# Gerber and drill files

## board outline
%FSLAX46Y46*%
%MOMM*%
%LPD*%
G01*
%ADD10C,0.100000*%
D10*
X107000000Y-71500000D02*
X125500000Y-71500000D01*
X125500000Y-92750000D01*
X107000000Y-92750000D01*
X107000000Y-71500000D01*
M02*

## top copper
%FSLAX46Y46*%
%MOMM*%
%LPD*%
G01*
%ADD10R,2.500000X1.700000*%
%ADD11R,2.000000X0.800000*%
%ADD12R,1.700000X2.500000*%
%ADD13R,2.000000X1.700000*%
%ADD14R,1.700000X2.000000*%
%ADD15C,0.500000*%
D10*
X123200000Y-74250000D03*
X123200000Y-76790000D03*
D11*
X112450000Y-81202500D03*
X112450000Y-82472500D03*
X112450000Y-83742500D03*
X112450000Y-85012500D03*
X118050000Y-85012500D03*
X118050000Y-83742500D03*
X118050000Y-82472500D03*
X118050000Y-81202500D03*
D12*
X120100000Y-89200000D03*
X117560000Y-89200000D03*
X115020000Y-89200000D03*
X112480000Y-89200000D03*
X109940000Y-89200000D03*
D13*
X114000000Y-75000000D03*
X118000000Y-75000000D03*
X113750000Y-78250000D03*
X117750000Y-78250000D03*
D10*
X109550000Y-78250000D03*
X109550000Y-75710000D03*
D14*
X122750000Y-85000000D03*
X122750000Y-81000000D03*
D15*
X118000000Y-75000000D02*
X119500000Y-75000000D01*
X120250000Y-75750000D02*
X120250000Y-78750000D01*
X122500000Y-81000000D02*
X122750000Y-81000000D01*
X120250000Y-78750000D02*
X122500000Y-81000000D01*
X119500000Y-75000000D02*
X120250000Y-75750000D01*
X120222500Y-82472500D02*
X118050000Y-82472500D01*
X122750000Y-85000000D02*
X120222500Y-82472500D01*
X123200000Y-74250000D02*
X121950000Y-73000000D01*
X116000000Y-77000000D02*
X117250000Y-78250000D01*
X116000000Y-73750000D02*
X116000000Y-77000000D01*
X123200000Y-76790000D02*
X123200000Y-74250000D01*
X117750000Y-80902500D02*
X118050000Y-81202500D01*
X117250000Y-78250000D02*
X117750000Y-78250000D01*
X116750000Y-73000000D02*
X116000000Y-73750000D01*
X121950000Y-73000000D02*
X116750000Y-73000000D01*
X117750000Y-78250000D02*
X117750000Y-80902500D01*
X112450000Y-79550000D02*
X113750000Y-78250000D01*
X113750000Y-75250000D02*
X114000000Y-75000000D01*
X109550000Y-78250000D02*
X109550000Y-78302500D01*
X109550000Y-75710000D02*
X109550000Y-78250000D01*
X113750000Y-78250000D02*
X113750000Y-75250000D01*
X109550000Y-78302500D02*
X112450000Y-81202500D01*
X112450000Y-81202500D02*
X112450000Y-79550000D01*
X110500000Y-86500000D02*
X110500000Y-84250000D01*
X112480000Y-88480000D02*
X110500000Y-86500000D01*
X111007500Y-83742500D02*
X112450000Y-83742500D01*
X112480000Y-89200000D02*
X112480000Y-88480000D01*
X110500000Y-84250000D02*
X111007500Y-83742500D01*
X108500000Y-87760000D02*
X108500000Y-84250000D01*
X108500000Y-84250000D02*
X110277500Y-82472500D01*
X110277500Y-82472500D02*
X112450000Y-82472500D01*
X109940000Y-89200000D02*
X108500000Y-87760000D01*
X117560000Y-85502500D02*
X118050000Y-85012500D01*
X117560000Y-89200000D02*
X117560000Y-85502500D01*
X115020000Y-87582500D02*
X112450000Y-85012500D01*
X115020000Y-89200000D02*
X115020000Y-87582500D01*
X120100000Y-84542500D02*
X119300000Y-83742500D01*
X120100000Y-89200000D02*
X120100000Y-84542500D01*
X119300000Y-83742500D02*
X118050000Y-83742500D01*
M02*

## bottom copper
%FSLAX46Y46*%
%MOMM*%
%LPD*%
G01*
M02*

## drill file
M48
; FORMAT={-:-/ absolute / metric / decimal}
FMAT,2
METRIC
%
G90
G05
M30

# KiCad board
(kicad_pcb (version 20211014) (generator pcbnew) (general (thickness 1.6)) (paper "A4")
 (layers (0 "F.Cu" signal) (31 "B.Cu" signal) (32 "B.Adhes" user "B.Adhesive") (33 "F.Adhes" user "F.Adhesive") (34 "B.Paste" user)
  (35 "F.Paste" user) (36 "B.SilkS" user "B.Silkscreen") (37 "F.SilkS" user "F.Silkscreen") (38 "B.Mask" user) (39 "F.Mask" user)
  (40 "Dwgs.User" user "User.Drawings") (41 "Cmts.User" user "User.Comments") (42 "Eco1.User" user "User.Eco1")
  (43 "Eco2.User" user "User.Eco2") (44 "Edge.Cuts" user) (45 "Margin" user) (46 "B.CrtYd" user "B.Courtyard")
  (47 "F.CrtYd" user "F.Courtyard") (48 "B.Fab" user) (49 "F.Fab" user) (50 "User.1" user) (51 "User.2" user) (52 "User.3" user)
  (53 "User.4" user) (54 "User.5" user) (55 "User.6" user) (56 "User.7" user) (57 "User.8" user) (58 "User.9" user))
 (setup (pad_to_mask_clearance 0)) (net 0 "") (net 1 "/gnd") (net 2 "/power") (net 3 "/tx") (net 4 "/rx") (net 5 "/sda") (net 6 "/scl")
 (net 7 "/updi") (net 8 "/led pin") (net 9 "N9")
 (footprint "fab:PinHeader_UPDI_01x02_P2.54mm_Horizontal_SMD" (layer "F.Cu") (at 123.2 74.25)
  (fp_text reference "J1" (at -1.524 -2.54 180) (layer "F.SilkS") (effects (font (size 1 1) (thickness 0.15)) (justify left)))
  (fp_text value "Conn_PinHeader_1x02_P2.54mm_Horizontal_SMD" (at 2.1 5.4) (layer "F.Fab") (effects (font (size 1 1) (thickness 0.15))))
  (pad "1" smd rect locked (at 0 0) (size 2.5 1.7) (layers "F.Cu" "F.Paste" "F.Mask") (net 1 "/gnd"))
  (pad "2" smd rect locked (at 0 2.54) (size 2.5 1.7) (layers "F.Cu" "F.Paste" "F.Mask") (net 1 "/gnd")))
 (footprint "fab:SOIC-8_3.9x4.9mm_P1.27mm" (layer "F.Cu") (at 115.25 83.1075)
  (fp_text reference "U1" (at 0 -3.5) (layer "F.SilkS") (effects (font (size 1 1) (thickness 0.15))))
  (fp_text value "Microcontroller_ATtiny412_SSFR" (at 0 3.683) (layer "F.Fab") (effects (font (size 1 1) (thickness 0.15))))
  (pad "1" smd rect locked (at -2.8 -1.905) (size 2 0.8) (layers "F.Cu" "F.Paste" "F.Mask") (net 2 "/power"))
  (pad "2" smd rect locked (at -2.8 -0.635) (size 2 0.8) (layers "F.Cu" "F.Paste" "F.Mask") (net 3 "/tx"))
  (pad "3" smd rect locked (at -2.8 0.635) (size 2 0.8) (layers "F.Cu" "F.Paste" "F.Mask") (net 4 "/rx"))
  (pad "4" smd rect locked (at -2.8 1.905) (size 2 0.8) (layers "F.Cu" "F.Paste" "F.Mask") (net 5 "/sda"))
  (pad "5" smd rect locked (at 2.8 1.905) (size 2 0.8) (layers "F.Cu" "F.Paste" "F.Mask") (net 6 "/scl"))
  (pad "6" smd rect locked (at 2.8 0.635) (size 2 0.8) (layers "F.Cu" "F.Paste" "F.Mask") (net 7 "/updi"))
  (pad "7" smd rect locked (at 2.8 -0.635) (size 2 0.8) (layers "F.Cu" "F.Paste" "F.Mask") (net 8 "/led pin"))
  (pad "8" smd rect locked (at 2.8 -1.905) (size 2 0.8) (layers "F.Cu" "F.Paste" "F.Mask") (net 1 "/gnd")))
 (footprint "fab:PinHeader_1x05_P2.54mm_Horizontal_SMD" (layer "F.Cu") (at 120.1 89.2 -90)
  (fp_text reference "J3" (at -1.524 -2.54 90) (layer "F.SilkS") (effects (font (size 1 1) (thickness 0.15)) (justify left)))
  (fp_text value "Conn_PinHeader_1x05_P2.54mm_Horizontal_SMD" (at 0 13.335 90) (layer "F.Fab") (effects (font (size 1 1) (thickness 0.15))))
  (pad "1" smd rect locked (at 0 0 270) (size 2.5 1.7) (layers "F.Cu" "F.Paste" "F.Mask") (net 7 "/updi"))
  (pad "2" smd rect locked (at 0 2.54 270) (size 2.5 1.7) (layers "F.Cu" "F.Paste" "F.Mask") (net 6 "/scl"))
  (pad "3" smd rect locked (at 0 5.08 270) (size 2.5 1.7) (layers "F.Cu" "F.Paste" "F.Mask") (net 5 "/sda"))
  (pad "4" smd rect locked (at 0 7.62 270) (size 2.5 1.7) (layers "F.Cu" "F.Paste" "F.Mask") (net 4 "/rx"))
  (pad "5" smd rect locked (at 0 10.16 270) (size 2.5 1.7) (layers "F.Cu" "F.Paste" "F.Mask") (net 3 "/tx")))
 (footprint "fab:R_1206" (layer "F.Cu") (at 116 75)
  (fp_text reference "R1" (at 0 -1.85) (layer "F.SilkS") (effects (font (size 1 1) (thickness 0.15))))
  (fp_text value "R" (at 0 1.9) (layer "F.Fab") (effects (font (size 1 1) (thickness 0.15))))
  (pad "1" smd rect locked (at -2 0) (size 2 1.7) (layers "F.Cu" "F.Paste" "F.Mask") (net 2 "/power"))
  (pad "2" smd rect locked (at 2 0) (size 2 1.7) (layers "F.Cu" "F.Paste" "F.Mask") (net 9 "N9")))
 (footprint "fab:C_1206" (layer "F.Cu") (at 115.75 78.25)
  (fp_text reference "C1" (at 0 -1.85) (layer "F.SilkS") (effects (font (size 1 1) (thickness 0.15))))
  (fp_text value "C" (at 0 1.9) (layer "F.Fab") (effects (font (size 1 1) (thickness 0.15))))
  (pad "1" smd rect locked (at -2 0) (size 2 1.7) (layers "F.Cu" "F.Paste" "F.Mask") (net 2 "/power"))
  (pad "2" smd rect locked (at 2 0) (size 2 1.7) (layers "F.Cu" "F.Paste" "F.Mask") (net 1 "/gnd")))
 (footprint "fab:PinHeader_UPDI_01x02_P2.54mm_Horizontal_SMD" (layer "F.Cu") (at 109.55 78.25 180)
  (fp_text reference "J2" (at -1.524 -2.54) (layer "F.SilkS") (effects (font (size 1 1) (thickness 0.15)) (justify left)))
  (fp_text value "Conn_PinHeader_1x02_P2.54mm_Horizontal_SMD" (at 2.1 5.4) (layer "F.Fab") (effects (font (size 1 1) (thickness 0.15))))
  (pad "1" smd rect locked (at 0 0 180) (size 2.5 1.7) (layers "F.Cu" "F.Paste" "F.Mask") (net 2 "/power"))
  (pad "2" smd rect locked (at 0 2.54 180) (size 2.5 1.7) (layers "F.Cu" "F.Paste" "F.Mask") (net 2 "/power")))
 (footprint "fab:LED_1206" (layer "F.Cu") (at 122.75 83 90)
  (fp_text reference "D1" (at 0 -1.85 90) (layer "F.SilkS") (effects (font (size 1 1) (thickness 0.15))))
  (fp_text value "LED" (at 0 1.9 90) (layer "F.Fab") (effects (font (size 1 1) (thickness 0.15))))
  (pad "1" smd rect locked (at -2 0 90) (size 2 1.7) (layers "F.Cu" "F.Paste" "F.Mask") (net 8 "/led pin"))
  (pad "2" smd rect locked (at 2 0 90) (size 2 1.7) (layers "F.Cu" "F.Paste" "F.Mask") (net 9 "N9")))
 (gr_rect (start 125.5 92.75) (end 107 71.5) (layer "Edge.Cuts") (width 0.1) (fill none))
 (segment (start 118 75) (end 119.5 75) (width 0.5) (layer "F.Cu") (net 9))
 (segment (start 120.25 75.75) (end 120.25 78.75) (width 0.5) (layer "F.Cu") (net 9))
 (segment (start 122.5 81) (end 122.75 81) (width 0.5) (layer "F.Cu") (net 9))
 (segment (start 120.25 78.75) (end 122.5 81) (width 0.5) (layer "F.Cu") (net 9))
 (segment (start 119.5 75) (end 120.25 75.75) (width 0.5) (layer "F.Cu") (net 9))
 (segment (start 120.2225 82.4725) (end 118.05 82.4725) (width 0.5) (layer "F.Cu") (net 8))
 (segment (start 122.75 85) (end 120.2225 82.4725) (width 0.5) (layer "F.Cu") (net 8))
 (segment (start 123.2 74.25) (end 121.95 73) (width 0.5) (layer "F.Cu") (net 1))
 (segment (start 116 77) (end 117.25 78.25) (width 0.5) (layer "F.Cu") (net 1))
 (segment (start 116 73.75) (end 116 77) (width 0.5) (layer "F.Cu") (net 1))
 (segment (start 123.2 76.79) (end 123.2 74.25) (width 0.5) (layer "F.Cu") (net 1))
 (segment (start 117.75 80.9025) (end 118.05 81.2025) (width 0.5) (layer "F.Cu") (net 1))
 (segment (start 117.25 78.25) (end 117.75 78.25) (width 0.5) (layer "F.Cu") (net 1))
 (segment (start 116.75 73) (end 116 73.75) (width 0.5) (layer "F.Cu") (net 1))
 (segment (start 121.95 73) (end 116.75 73) (width 0.5) (layer "F.Cu") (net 1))
 (segment (start 117.75 78.25) (end 117.75 80.9025) (width 0.5) (layer "F.Cu") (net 1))
 (segment (start 112.45 79.55) (end 113.75 78.25) (width 0.5) (layer "F.Cu") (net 2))
 (segment (start 113.75 75.25) (end 114 75) (width 0.5) (layer "F.Cu") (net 2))
 (segment (start 109.55 78.25) (end 109.55 78.3025) (width 0.5) (layer "F.Cu") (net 2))
 (segment (start 109.55 75.71) (end 109.55 78.25) (width 0.5) (layer "F.Cu") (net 2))
 (segment (start 113.75 78.25) (end 113.75 75.25) (width 0.5) (layer "F.Cu") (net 2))
 (segment (start 109.55 78.3025) (end 112.45 81.2025) (width 0.5) (layer "F.Cu") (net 2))
 (segment (start 112.45 81.2025) (end 112.45 79.55) (width 0.5) (layer "F.Cu") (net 2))
 (segment (start 110.5 86.5) (end 110.5 84.25) (width 0.5) (layer "F.Cu") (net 4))
 (segment (start 112.48 88.48) (end 110.5 86.5) (width 0.5) (layer "F.Cu") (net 4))
 (segment (start 111.0075 83.7425) (end 112.45 83.7425) (width 0.5) (layer "F.Cu") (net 4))
 (segment (start 112.48 89.2) (end 112.48 88.48) (width 0.5) (layer "F.Cu") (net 4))
 (segment (start 110.5 84.25) (end 111.0075 83.7425) (width 0.5) (layer "F.Cu") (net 4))
 (segment (start 108.5 87.76) (end 108.5 84.25) (width 0.5) (layer "F.Cu") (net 3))
 (segment (start 108.5 84.25) (end 110.2775 82.4725) (width 0.5) (layer "F.Cu") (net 3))
 (segment (start 110.2775 82.4725) (end 112.45 82.4725) (width 0.5) (layer "F.Cu") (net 3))
 (segment (start 109.94 89.2) (end 108.5 87.76) (width 0.5) (layer "F.Cu") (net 3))
 (segment (start 117.56 85.5025) (end 118.05 85.0125) (width 0.5) (layer "F.Cu") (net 6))
 (segment (start 117.56 89.2) (end 117.56 85.5025) (width 0.5) (layer "F.Cu") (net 6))
 (segment (start 115.02 87.5825) (end 112.45 85.0125) (width 0.5) (layer "F.Cu") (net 5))
 (segment (start 115.02 89.2) (end 115.02 87.5825) (width 0.5) (layer "F.Cu") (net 5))
 (segment (start 120.1 84.5425) (end 119.3 83.7425) (width 0.5) (layer "F.Cu") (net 7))
 (segment (start 120.1 89.2) (end 120.1 84.5425) (width 0.5) (layer "F.Cu") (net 7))
 (segment (start 119.3 83.7425) (end 118.05 83.7425) (width 0.5) (layer "F.Cu") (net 7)))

